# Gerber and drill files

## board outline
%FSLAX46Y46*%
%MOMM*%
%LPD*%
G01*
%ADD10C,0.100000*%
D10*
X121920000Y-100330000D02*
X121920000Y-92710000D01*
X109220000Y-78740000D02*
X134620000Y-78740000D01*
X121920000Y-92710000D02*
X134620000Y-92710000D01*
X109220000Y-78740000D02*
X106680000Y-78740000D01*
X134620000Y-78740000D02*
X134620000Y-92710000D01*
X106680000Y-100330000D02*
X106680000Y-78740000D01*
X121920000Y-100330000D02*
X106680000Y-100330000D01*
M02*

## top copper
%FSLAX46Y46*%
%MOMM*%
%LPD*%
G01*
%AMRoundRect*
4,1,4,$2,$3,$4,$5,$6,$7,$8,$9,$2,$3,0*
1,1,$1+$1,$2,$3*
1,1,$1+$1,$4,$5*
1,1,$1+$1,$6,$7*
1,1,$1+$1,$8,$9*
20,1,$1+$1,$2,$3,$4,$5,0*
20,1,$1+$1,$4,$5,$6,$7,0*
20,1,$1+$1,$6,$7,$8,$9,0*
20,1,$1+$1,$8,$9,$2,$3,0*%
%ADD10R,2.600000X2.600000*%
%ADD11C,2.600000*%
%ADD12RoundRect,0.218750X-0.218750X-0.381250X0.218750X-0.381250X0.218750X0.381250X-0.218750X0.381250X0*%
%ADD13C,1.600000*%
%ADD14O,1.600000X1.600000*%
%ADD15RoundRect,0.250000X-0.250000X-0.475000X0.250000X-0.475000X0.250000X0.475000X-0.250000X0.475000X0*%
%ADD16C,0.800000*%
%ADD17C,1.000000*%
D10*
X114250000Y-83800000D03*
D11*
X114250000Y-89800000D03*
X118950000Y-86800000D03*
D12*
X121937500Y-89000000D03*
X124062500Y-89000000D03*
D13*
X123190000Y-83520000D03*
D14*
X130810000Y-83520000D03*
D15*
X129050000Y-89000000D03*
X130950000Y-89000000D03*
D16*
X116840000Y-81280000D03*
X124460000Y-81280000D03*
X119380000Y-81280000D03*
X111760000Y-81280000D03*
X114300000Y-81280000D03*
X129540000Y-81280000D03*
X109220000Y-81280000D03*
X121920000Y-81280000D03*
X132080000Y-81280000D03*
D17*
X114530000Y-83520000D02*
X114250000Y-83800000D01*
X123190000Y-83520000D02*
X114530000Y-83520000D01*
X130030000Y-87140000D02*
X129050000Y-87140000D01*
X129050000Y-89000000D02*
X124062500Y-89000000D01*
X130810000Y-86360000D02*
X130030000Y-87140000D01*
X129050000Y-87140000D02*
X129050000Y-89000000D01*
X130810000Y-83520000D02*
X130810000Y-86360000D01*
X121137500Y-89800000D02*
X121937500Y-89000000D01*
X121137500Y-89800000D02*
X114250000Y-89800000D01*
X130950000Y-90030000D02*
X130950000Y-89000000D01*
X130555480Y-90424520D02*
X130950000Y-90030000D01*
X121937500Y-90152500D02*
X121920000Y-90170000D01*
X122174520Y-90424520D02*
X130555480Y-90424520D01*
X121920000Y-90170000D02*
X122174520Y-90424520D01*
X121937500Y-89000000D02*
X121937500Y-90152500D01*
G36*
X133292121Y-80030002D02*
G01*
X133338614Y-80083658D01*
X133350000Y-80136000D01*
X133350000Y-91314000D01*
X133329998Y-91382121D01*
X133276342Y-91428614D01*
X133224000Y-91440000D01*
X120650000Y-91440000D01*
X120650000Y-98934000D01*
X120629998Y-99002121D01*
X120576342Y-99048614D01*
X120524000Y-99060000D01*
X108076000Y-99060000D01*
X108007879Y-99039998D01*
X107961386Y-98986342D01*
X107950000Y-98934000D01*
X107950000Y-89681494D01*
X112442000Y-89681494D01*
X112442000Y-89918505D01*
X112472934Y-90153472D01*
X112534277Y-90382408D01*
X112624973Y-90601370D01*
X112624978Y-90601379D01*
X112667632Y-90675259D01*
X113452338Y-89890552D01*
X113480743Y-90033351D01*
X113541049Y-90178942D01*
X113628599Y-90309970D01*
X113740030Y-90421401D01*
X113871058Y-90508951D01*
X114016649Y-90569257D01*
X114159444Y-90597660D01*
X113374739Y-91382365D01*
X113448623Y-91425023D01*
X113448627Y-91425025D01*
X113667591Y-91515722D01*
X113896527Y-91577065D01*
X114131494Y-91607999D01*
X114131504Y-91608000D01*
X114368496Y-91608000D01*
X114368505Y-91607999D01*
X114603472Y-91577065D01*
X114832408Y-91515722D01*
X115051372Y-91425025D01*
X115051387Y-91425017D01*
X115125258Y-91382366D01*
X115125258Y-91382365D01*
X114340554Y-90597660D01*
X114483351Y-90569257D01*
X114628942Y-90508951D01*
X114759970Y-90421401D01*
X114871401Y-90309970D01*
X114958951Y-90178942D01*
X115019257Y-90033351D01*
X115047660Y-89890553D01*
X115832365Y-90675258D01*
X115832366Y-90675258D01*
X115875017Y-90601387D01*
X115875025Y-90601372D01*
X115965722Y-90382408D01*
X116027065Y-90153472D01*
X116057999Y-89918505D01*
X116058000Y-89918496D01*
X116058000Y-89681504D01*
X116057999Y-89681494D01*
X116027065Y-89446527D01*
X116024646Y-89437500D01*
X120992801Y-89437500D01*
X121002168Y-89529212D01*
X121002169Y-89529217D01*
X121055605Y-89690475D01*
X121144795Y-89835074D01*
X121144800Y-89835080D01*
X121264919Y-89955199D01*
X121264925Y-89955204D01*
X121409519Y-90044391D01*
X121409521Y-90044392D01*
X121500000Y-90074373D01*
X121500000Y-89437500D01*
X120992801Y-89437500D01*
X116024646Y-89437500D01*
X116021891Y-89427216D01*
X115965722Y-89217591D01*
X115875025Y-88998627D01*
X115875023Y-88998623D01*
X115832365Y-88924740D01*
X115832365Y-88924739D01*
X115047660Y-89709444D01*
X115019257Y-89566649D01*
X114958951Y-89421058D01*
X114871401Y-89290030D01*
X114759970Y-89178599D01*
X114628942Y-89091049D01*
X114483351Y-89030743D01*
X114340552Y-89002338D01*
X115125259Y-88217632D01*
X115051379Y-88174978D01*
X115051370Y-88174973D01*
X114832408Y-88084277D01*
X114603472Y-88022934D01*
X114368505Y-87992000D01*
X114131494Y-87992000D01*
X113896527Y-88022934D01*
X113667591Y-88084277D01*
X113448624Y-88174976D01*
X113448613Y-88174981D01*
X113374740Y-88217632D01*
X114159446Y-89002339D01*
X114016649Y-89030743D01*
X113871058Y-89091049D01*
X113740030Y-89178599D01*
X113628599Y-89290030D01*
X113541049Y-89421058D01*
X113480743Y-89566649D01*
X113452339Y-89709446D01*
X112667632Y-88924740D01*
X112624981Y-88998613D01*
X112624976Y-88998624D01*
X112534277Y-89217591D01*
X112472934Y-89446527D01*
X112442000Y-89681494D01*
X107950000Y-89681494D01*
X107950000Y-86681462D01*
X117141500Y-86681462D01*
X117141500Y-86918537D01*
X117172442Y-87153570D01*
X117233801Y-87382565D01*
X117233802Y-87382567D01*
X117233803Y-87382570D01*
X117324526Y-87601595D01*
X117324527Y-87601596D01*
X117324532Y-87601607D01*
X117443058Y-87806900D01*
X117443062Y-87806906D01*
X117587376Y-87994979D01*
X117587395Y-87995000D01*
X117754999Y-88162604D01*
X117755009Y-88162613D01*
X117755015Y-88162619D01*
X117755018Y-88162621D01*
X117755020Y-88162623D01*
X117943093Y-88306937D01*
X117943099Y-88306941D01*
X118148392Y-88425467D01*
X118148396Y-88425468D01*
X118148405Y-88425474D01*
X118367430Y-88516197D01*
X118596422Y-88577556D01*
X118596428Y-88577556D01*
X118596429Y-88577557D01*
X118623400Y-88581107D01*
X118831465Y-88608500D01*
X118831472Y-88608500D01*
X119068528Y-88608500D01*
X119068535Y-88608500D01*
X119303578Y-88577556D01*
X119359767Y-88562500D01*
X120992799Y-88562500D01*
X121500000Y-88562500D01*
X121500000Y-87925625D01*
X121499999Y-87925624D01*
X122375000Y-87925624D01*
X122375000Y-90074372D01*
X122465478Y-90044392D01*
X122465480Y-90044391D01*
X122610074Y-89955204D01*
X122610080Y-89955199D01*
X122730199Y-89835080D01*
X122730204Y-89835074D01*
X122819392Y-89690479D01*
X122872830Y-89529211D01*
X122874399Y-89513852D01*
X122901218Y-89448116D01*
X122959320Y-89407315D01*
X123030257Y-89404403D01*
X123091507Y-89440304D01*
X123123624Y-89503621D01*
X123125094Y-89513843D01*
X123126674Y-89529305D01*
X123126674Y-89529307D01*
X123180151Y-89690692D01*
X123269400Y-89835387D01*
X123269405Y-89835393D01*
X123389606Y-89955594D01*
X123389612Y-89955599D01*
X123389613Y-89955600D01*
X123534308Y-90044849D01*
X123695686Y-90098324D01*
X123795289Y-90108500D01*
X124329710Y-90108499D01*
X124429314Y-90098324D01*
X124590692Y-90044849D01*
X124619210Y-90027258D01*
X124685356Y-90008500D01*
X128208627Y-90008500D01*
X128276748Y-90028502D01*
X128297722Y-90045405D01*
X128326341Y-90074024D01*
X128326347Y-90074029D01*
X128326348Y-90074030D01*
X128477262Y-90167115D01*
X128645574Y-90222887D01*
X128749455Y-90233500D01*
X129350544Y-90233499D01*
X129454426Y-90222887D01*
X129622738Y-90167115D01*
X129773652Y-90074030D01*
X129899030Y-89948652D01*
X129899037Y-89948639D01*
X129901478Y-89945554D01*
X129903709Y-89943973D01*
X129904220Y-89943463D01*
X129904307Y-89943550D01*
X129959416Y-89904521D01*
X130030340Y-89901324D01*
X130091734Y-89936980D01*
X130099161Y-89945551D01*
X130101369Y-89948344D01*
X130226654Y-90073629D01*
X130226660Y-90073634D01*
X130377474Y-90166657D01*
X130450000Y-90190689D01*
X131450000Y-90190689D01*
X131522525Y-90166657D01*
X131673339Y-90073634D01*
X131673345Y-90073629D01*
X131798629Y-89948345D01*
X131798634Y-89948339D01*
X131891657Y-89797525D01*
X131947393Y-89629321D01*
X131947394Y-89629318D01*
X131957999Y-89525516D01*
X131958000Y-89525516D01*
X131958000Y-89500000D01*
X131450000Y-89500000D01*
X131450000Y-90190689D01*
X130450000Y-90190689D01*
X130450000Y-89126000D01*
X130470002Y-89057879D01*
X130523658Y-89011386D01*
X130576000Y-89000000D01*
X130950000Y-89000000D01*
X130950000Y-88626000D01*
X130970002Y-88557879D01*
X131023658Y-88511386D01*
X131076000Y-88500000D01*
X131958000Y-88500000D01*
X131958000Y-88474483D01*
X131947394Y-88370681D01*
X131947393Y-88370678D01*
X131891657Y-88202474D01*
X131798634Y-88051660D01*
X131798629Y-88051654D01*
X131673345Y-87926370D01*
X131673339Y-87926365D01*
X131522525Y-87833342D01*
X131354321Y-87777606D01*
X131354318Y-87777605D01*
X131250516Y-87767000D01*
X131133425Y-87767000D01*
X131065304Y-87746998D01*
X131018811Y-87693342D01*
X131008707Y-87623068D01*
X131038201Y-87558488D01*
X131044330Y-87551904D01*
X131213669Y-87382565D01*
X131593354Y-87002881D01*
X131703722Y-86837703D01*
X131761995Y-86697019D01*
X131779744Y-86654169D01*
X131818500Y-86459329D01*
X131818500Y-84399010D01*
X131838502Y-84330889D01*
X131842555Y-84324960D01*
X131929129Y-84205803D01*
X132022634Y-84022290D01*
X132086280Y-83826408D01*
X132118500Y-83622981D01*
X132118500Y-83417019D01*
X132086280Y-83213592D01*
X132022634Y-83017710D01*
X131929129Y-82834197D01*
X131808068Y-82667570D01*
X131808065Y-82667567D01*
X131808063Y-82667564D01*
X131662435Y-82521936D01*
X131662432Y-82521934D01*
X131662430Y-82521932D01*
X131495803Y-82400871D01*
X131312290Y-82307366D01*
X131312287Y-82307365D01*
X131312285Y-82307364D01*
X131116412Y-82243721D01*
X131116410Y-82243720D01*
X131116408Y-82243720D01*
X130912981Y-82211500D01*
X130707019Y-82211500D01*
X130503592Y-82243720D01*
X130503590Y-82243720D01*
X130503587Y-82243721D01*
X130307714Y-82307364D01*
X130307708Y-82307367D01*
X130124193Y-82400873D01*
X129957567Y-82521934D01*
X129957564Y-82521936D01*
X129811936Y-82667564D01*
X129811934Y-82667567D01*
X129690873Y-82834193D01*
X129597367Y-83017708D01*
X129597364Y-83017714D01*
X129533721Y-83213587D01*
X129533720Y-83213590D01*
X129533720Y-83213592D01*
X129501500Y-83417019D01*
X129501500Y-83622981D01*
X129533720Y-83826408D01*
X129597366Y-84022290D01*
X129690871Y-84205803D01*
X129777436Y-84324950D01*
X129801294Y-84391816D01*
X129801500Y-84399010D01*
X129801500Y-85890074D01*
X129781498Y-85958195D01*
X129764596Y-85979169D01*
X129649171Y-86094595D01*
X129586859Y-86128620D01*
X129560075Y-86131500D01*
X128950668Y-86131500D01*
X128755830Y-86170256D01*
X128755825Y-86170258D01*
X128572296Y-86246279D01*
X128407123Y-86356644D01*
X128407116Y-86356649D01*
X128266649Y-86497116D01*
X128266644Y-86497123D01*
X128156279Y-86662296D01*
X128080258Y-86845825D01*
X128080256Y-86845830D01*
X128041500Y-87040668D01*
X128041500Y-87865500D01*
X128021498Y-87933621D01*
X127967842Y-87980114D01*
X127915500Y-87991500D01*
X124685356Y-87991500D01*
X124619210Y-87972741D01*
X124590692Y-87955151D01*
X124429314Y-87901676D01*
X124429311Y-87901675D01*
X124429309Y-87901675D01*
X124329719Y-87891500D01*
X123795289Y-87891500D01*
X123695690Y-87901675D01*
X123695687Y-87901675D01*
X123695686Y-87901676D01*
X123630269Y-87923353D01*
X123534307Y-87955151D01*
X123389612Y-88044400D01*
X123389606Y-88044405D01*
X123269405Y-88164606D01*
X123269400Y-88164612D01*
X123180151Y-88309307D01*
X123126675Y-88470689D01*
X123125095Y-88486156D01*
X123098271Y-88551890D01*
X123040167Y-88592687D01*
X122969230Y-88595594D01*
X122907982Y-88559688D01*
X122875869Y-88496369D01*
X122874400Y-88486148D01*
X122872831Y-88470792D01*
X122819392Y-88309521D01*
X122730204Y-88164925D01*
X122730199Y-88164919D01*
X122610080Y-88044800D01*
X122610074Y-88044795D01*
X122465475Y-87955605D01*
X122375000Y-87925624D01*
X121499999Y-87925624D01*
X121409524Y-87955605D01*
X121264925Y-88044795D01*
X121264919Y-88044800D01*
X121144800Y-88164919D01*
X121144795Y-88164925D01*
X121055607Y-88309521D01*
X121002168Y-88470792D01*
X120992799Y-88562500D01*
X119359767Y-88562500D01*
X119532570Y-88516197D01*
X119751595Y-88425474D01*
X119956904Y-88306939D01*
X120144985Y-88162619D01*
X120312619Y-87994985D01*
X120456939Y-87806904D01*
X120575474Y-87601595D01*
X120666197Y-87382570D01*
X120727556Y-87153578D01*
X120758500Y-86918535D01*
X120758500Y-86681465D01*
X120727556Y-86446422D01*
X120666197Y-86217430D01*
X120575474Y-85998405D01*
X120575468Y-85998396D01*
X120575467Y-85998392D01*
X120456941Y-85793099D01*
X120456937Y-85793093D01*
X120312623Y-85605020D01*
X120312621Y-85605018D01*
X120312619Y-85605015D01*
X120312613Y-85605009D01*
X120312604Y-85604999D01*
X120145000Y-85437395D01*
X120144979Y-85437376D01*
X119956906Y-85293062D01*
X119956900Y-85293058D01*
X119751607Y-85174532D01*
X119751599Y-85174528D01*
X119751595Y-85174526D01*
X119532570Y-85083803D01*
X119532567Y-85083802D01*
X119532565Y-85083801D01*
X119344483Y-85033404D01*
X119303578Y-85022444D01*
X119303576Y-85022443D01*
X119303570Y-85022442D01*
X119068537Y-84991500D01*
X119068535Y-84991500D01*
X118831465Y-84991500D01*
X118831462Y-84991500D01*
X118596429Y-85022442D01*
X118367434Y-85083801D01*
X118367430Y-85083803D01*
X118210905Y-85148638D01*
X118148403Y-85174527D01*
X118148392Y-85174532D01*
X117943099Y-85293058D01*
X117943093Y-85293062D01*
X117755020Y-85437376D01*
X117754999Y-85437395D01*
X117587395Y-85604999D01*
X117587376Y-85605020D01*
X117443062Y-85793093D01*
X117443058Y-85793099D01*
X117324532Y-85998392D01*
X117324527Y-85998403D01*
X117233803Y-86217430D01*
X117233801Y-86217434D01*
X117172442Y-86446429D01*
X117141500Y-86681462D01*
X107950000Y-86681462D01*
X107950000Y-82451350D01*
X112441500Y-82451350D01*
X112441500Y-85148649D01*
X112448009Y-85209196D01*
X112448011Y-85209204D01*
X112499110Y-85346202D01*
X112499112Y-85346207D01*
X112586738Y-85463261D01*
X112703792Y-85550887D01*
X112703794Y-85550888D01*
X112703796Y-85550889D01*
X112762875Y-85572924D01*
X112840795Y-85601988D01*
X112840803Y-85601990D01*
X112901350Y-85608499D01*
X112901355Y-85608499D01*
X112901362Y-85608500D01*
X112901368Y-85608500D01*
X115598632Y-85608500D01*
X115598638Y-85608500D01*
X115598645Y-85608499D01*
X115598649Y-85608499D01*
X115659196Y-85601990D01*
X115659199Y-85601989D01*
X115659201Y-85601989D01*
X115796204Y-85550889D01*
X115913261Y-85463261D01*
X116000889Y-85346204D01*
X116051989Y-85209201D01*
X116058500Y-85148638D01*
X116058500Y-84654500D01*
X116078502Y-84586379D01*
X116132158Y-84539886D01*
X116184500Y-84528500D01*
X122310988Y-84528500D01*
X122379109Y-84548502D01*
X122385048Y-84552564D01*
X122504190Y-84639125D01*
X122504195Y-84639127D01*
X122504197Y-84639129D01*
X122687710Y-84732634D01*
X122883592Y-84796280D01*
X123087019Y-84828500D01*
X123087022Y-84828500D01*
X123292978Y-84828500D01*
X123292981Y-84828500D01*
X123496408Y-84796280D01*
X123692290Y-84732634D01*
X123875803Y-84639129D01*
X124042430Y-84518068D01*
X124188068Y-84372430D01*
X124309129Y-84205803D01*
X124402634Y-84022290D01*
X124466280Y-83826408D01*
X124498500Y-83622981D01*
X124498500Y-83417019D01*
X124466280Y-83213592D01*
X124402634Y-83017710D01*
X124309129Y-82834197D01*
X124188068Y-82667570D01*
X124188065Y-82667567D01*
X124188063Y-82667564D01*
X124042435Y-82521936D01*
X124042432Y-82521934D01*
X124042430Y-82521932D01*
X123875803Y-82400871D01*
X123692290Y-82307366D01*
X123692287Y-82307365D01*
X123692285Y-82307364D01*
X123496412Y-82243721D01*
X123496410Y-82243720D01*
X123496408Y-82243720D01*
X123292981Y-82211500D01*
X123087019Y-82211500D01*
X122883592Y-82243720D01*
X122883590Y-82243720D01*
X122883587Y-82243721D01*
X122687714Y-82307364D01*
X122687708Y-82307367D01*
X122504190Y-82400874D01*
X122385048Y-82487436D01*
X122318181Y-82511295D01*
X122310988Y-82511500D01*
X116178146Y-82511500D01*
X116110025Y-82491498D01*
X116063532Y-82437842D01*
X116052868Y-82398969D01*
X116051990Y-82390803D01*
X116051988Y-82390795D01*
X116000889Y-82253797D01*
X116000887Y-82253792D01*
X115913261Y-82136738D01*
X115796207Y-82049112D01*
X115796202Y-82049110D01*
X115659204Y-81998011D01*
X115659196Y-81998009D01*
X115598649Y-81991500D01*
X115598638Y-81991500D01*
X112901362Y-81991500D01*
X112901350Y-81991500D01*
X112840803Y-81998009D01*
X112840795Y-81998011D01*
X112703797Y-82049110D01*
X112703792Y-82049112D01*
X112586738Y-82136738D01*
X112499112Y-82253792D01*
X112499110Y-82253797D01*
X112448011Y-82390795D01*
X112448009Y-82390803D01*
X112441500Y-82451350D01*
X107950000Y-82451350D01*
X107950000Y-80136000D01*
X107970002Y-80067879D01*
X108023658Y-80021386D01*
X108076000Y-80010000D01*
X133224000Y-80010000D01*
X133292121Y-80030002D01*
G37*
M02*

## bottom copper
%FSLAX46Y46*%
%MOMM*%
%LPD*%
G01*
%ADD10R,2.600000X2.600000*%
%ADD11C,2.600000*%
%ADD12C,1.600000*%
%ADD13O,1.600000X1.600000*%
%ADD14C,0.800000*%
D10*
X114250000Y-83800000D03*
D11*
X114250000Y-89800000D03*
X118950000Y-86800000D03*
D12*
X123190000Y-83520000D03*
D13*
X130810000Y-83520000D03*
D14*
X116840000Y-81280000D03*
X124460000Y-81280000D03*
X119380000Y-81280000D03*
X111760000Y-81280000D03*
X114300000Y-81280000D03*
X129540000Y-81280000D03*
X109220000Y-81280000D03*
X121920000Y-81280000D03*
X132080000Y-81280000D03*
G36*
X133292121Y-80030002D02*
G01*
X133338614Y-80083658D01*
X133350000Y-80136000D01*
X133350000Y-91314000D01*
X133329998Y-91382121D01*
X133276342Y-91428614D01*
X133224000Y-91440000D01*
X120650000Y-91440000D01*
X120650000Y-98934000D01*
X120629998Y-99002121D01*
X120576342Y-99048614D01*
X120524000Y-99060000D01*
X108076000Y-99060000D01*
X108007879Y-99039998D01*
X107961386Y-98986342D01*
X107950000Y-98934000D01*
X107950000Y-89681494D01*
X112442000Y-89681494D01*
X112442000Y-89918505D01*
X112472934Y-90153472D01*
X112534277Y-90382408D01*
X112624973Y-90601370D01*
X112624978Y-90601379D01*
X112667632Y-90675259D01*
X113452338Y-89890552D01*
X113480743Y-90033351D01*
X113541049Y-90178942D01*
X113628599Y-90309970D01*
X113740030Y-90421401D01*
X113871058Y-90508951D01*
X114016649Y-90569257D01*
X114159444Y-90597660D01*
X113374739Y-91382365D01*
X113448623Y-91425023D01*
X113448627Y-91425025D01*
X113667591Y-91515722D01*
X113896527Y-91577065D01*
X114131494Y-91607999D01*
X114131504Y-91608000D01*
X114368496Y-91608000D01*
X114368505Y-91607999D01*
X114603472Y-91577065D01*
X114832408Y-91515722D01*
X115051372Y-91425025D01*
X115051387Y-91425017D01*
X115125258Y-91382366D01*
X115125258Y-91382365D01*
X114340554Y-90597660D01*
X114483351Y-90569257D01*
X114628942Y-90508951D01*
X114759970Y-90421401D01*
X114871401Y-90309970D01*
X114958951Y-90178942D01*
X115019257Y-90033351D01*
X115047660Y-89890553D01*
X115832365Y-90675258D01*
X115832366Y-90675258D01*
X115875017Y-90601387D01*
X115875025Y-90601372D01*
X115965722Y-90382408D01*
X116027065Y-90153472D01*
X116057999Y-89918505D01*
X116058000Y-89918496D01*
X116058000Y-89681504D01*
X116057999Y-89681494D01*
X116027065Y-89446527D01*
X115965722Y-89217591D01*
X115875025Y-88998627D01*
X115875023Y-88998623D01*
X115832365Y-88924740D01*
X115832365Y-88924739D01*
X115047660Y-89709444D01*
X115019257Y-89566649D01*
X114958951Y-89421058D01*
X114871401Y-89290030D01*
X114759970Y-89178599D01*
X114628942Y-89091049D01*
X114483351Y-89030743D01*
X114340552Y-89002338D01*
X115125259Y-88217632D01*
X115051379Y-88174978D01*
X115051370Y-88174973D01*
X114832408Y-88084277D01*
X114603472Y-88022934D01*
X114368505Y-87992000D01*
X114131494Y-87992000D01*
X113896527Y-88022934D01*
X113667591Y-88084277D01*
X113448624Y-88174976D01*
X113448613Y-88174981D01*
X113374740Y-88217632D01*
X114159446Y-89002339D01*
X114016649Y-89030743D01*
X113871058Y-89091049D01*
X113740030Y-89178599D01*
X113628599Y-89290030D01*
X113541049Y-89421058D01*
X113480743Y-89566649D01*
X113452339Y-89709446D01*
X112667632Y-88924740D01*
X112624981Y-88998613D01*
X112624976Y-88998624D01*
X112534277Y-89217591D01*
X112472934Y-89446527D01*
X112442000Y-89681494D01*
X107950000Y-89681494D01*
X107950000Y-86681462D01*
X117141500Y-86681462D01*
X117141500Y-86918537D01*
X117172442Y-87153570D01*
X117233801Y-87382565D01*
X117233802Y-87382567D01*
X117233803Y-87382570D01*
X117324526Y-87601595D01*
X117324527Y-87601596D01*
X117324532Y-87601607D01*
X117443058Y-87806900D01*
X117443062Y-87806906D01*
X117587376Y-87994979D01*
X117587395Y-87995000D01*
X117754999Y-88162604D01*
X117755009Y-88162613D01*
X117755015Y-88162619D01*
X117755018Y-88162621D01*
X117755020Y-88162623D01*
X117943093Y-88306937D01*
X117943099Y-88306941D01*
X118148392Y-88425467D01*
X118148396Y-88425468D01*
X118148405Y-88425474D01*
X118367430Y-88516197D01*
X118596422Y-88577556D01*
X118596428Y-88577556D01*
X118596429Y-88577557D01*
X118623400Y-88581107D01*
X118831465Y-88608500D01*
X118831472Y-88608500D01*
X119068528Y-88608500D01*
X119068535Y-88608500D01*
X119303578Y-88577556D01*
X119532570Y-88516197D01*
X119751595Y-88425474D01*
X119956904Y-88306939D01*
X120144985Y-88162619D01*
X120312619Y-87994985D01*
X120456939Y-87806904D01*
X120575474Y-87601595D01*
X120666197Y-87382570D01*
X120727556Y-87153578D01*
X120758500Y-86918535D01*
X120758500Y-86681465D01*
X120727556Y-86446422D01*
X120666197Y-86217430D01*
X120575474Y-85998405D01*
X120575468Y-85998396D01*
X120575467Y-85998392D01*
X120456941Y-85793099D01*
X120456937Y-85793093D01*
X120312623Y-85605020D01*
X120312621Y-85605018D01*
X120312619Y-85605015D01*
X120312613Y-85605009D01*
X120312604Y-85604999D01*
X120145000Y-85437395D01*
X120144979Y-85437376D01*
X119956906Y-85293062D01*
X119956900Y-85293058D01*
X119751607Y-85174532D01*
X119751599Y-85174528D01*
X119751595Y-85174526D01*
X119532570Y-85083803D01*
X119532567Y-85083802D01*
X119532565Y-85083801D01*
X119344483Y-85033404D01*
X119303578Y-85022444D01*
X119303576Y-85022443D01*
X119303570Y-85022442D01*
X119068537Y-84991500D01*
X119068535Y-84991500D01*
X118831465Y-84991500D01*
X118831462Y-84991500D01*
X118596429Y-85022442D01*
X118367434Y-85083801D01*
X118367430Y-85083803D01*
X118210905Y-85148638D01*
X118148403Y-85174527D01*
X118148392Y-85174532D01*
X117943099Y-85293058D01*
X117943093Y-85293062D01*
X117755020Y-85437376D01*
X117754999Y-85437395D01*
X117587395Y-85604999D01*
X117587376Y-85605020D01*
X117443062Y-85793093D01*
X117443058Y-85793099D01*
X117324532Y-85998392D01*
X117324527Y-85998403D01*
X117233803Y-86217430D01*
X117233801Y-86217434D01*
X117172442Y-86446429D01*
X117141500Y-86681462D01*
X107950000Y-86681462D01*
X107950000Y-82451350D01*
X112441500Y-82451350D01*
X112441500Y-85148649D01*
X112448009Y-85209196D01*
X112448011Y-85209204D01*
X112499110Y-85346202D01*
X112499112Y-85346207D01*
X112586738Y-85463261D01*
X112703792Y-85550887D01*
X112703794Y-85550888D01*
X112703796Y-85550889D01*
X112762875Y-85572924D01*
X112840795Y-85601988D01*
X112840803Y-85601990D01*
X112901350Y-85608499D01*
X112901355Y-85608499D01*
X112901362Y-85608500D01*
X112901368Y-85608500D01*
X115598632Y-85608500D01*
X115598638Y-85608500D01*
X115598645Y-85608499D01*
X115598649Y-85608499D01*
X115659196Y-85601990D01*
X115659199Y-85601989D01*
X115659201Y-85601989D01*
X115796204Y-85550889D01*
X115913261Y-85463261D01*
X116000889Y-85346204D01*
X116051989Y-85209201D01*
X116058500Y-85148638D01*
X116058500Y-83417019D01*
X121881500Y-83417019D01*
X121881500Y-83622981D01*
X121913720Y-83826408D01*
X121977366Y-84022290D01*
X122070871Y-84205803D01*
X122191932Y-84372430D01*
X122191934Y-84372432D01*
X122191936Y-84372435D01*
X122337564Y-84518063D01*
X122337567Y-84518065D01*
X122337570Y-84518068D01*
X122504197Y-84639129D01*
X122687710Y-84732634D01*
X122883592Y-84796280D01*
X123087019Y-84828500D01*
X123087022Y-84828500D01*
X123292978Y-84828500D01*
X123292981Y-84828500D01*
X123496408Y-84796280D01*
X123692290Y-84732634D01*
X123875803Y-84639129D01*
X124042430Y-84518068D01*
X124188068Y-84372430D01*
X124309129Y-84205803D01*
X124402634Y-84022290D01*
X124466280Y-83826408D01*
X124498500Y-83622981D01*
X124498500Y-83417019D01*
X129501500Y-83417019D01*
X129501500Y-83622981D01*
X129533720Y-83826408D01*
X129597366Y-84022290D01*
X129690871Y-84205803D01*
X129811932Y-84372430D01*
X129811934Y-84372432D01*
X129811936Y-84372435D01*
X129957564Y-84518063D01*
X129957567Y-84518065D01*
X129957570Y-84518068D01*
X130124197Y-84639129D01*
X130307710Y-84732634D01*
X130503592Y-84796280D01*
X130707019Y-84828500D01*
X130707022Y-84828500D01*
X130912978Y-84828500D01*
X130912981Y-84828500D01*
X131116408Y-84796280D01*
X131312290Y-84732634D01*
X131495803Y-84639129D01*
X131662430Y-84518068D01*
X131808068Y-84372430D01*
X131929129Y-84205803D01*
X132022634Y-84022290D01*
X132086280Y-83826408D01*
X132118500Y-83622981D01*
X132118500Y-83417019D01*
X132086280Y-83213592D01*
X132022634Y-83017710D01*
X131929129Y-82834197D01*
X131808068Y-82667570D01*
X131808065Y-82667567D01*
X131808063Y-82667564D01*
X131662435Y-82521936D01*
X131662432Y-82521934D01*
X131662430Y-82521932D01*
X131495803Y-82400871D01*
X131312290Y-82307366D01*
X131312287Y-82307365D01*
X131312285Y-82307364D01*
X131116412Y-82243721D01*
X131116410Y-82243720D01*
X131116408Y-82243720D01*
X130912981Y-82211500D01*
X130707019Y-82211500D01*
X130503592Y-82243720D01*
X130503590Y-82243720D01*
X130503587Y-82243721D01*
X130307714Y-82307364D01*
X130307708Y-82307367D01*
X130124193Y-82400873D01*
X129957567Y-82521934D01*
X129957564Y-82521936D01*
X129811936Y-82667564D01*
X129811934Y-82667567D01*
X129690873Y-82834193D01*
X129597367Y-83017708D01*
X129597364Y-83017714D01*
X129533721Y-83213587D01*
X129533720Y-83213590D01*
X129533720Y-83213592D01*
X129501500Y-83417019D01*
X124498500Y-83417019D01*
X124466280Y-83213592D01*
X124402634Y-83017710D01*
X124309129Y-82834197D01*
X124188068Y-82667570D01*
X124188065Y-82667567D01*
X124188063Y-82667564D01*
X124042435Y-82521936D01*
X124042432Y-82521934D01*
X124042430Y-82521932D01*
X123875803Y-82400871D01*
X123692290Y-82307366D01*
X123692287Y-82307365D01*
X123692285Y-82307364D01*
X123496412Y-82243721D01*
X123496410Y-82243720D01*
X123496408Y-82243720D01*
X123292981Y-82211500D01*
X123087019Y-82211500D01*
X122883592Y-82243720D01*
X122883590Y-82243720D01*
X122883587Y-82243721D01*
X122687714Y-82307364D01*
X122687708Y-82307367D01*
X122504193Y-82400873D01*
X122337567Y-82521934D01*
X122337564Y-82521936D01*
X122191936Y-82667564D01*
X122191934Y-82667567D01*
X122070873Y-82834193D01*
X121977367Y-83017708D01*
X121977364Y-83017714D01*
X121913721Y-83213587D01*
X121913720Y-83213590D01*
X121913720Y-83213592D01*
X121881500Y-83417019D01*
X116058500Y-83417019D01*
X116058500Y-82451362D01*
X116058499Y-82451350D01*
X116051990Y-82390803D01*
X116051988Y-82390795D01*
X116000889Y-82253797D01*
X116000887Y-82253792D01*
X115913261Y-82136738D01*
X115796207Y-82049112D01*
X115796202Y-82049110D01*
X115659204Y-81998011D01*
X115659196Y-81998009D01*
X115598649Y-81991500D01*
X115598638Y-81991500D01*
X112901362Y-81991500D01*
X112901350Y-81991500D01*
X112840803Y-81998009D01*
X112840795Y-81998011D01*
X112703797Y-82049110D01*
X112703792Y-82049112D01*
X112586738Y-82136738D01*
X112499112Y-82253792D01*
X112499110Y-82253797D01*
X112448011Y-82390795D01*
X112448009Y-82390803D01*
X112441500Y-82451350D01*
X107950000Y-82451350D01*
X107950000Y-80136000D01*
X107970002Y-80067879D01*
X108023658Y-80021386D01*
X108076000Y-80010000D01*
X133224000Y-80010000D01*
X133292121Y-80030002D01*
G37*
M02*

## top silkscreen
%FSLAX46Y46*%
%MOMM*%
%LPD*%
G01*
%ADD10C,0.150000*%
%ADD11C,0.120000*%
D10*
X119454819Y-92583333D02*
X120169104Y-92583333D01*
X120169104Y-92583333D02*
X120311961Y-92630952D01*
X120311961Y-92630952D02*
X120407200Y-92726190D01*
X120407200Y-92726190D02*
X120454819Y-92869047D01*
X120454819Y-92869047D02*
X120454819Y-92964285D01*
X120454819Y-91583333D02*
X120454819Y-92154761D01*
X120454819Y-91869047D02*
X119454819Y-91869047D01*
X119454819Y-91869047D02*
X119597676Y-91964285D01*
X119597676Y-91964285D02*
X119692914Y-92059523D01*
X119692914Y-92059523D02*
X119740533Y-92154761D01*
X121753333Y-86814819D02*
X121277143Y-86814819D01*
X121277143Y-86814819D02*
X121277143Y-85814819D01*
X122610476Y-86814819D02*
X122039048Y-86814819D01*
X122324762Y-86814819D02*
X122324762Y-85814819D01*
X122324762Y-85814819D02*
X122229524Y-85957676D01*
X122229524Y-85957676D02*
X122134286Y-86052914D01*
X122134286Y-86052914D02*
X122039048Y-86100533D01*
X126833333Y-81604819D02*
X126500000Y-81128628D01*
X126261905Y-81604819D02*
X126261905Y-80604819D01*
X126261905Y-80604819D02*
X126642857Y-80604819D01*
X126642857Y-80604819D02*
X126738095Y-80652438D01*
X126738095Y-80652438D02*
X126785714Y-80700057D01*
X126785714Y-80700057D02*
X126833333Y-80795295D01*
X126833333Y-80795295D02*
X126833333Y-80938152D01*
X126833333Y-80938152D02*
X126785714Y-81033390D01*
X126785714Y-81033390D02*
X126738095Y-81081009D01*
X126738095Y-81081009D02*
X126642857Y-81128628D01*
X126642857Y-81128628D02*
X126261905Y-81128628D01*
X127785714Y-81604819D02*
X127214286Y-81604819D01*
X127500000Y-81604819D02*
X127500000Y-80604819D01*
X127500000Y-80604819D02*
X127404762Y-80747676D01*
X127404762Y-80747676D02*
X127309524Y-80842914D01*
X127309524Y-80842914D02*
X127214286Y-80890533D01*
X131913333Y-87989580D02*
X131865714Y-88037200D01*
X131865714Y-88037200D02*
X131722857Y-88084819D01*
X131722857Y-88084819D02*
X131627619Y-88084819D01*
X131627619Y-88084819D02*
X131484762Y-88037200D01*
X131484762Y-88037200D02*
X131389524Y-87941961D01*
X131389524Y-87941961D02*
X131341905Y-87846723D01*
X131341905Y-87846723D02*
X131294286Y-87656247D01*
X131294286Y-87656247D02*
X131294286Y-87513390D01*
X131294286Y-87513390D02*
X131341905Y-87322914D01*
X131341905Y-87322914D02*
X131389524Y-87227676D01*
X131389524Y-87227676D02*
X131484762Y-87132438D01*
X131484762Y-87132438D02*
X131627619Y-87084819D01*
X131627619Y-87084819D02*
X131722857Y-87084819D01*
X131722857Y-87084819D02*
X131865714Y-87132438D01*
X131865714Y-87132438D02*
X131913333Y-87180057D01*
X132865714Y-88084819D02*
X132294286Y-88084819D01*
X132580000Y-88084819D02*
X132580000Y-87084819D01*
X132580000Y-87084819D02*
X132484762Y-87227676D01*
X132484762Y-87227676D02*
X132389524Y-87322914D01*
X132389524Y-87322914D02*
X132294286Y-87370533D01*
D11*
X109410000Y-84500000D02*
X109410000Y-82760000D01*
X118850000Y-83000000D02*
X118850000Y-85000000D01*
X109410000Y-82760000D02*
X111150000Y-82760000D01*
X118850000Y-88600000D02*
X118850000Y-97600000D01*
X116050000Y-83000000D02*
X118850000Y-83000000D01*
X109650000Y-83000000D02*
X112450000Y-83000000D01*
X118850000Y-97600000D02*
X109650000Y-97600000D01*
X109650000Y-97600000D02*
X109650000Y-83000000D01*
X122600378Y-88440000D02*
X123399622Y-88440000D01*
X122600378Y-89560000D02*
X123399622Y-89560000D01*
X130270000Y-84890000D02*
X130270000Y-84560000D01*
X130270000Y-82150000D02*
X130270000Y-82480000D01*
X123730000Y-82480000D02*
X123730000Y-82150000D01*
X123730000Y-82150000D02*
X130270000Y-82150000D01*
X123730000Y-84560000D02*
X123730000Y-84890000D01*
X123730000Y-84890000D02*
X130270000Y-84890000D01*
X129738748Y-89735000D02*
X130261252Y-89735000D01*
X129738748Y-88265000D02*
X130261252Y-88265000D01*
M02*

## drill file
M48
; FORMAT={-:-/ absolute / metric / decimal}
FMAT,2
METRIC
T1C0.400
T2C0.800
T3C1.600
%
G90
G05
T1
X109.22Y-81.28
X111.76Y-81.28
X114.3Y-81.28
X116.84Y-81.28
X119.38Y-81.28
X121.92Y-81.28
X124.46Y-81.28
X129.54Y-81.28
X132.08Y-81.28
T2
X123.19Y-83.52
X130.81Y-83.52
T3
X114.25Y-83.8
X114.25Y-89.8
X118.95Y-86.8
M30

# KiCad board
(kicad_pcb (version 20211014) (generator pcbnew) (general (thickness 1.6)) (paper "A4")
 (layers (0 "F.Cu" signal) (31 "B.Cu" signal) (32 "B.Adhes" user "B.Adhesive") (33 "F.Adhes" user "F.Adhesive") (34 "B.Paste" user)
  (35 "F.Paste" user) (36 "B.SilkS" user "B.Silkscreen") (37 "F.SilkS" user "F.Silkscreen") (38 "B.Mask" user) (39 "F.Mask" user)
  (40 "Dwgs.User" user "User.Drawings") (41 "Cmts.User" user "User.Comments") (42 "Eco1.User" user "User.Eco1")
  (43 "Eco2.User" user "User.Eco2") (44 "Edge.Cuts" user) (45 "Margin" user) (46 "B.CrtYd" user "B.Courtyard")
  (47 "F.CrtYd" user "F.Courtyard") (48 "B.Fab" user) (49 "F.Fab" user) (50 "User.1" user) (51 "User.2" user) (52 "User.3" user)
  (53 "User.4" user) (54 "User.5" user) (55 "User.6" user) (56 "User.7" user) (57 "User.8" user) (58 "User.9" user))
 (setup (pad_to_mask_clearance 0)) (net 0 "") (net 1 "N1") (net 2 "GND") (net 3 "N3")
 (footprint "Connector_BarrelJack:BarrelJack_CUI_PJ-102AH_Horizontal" (layer "F.Cu") (at 114.25 83.8)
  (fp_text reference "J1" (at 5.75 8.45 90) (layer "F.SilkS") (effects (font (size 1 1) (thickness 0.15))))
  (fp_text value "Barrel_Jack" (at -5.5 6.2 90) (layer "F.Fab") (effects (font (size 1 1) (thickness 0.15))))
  (fp_line (start -4.84 0.7) (end -4.84 -1.04) (layer "F.SilkS") (width 0.12))
  (fp_line (start 4.6 -0.8) (end 4.6 1.2) (layer "F.SilkS") (width 0.12))
  (fp_line (start -4.84 -1.04) (end -3.1 -1.04) (layer "F.SilkS") (width 0.12))
  (fp_line (start 4.6 4.8) (end 4.6 13.8) (layer "F.SilkS") (width 0.12))
  (fp_line (start 1.8 -0.8) (end 4.6 -0.8) (layer "F.SilkS") (width 0.12))
  (fp_line (start -4.6 -0.8) (end -1.8 -0.8) (layer "F.SilkS") (width 0.12))
  (fp_line (start 4.6 13.8) (end -4.6 13.8) (layer "F.SilkS") (width 0.12))
  (fp_line (start -4.6 13.8) (end -4.6 -0.8) (layer "F.SilkS") (width 0.12))
  (pad "1" thru_hole rect (at 0 0) (size 2.6 2.6) (drill 1.6) (layers *.Cu *.Mask) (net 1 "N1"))
  (pad "2" thru_hole circle (at 0 6) (size 2.6 2.6) (drill 1.6) (layers *.Cu *.Mask) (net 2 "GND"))
  (pad "3" thru_hole circle (at 4.7 3) (size 2.6 2.6) (drill 1.6) (layers *.Cu *.Mask)))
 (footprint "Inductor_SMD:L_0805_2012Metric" (layer "F.Cu") (at 123 89)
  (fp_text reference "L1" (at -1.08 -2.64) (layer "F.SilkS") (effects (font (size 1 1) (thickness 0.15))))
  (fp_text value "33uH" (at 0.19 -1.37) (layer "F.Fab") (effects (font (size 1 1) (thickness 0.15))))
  (fp_line (start -0.399622 -0.56) (end 0.399622 -0.56) (layer "F.SilkS") (width 0.12))
  (fp_line (start -0.399622 0.56) (end 0.399622 0.56) (layer "F.SilkS") (width 0.12))
  (pad "1" smd roundrect (at -1.0625 0) (size 0.875 1.2) (layers "F.Cu" "F.Paste" "F.Mask") (roundrect_rratio 0.25) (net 2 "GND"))
  (pad "2" smd roundrect (at 1.0625 0) (size 0.875 1.2) (layers "F.Cu" "F.Paste" "F.Mask") (roundrect_rratio 0.25) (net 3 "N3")))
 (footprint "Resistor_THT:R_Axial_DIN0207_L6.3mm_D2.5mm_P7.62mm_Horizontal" (layer "F.Cu") (at 123.19 83.52)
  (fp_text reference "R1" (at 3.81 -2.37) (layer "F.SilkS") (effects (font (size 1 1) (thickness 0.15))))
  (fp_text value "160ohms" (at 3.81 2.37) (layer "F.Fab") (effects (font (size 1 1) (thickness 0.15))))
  (fp_line (start 7.08 1.37) (end 7.08 1.04) (layer "F.SilkS") (width 0.12))
  (fp_line (start 7.08 -1.37) (end 7.08 -1.04) (layer "F.SilkS") (width 0.12))
  (fp_line (start 0.54 -1.04) (end 0.54 -1.37) (layer "F.SilkS") (width 0.12))
  (fp_line (start 0.54 -1.37) (end 7.08 -1.37) (layer "F.SilkS") (width 0.12))
  (fp_line (start 0.54 1.04) (end 0.54 1.37) (layer "F.SilkS") (width 0.12))
  (fp_line (start 0.54 1.37) (end 7.08 1.37) (layer "F.SilkS") (width 0.12))
  (pad "1" thru_hole circle (at 0 0) (size 1.6 1.6) (drill 0.8) (layers *.Cu *.Mask) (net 1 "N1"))
  (pad "2" thru_hole oval (at 7.62 0) (size 1.6 1.6) (drill 0.8) (layers *.Cu *.Mask) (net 3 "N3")))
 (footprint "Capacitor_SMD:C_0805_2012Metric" (layer "F.Cu") (at 130 89)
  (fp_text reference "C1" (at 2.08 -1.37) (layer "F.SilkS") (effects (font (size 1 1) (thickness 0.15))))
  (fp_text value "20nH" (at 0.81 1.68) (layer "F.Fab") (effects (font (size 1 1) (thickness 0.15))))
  (fp_line (start -0.261252 0.735) (end 0.261252 0.735) (layer "F.SilkS") (width 0.12))
  (fp_line (start -0.261252 -0.735) (end 0.261252 -0.735) (layer "F.SilkS") (width 0.12))
  (pad "1" smd roundrect (at -0.95 0) (size 1 1.45) (layers "F.Cu" "F.Paste" "F.Mask") (roundrect_rratio 0.25) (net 3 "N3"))
  (pad "2" smd roundrect (at 0.95 0) (size 1 1.45) (layers "F.Cu" "F.Paste" "F.Mask") (roundrect_rratio 0.25) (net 2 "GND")))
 (gr_line (start 121.92 100.33) (end 121.92 92.71) (layer "Edge.Cuts") (width 0.1))
 (gr_line (start 109.22 78.74) (end 134.62 78.74) (layer "Edge.Cuts") (width 0.1))
 (gr_line (start 121.92 92.71) (end 134.62 92.71) (layer "Edge.Cuts") (width 0.1))
 (gr_line (start 109.22 78.74) (end 106.68 78.74) (layer "Edge.Cuts") (width 0.1))
 (gr_line (start 134.62 78.74) (end 134.62 92.71) (layer "Edge.Cuts") (width 0.1))
 (gr_line (start 106.68 100.33) (end 106.68 78.74) (layer "Edge.Cuts") (width 0.1))
 (gr_line (start 121.92 100.33) (end 106.68 100.33) (layer "Edge.Cuts") (width 0.1))
 (segment (start 114.53 83.52) (end 114.25 83.8) (width 1) (layer "F.Cu") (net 1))
 (segment (start 123.19 83.52) (end 114.53 83.52) (width 1) (layer "F.Cu") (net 1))
 (segment (start 130.03 87.14) (end 129.05 87.14) (width 1) (layer "F.Cu") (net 3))
 (segment (start 129.05 89) (end 124.0625 89) (width 1) (layer "F.Cu") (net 3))
 (segment (start 130.81 86.36) (end 130.03 87.14) (width 1) (layer "F.Cu") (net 3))
 (segment (start 129.05 87.14) (end 129.05 89) (width 1) (layer "F.Cu") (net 3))
 (segment (start 130.81 83.52) (end 130.81 86.36) (width 1) (layer "F.Cu") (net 3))
 (segment (start 121.1375 89.8) (end 121.9375 89) (width 1) (layer "F.Cu") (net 2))
 (segment (start 121.1375 89.8) (end 114.25 89.8) (width 1) (layer "F.Cu") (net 2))
 (segment (start 130.95 90.03) (end 130.95 89) (width 1) (layer "F.Cu") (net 2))
 (segment (start 130.55548 90.42452) (end 130.95 90.03) (width 1) (layer "F.Cu") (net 2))
 (segment (start 121.9375 90.1525) (end 121.92 90.17) (width 1) (layer "F.Cu") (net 2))
 (segment (start 122.17452 90.42452) (end 130.55548 90.42452) (width 1) (layer "F.Cu") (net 2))
 (segment (start 121.92 90.17) (end 122.17452 90.42452) (width 1) (layer "F.Cu") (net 2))
 (segment (start 121.9375 89) (end 121.9375 90.1525) (width 1) (layer "F.Cu") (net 2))
 (via (at 116.84 81.28) (size 0.8) (drill 0.4) (layers "F.Cu" "B.Cu") (free) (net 2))
 (via (at 124.46 81.28) (size 0.8) (drill 0.4) (layers "F.Cu" "B.Cu") (free) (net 2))
 (via (at 119.38 81.28) (size 0.8) (drill 0.4) (layers "F.Cu" "B.Cu") (free) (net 2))
 (via (at 111.76 81.28) (size 0.8) (drill 0.4) (layers "F.Cu" "B.Cu") (free) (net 2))
 (via (at 114.3 81.28) (size 0.8) (drill 0.4) (layers "F.Cu" "B.Cu") (free) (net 2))
 (via (at 129.54 81.28) (size 0.8) (drill 0.4) (layers "F.Cu" "B.Cu") (free) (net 2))
 (via (at 109.22 81.28) (size 0.8) (drill 0.4) (layers "F.Cu" "B.Cu") (free) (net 2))
 (via (at 121.92 81.28) (size 0.8) (drill 0.4) (layers "F.Cu" "B.Cu") (free) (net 2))
 (via (at 132.08 81.28) (size 0.8) (drill 0.4) (layers "F.Cu" "B.Cu") (free) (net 2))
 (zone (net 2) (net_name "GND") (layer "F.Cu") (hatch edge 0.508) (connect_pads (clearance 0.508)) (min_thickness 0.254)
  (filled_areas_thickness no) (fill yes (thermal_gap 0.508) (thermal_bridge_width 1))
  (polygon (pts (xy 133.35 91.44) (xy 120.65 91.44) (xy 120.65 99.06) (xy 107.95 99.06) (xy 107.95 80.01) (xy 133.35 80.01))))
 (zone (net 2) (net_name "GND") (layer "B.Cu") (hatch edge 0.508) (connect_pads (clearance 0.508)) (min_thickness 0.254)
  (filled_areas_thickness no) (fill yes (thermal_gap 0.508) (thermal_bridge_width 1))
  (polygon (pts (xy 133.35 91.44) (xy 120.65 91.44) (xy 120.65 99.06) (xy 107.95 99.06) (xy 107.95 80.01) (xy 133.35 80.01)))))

